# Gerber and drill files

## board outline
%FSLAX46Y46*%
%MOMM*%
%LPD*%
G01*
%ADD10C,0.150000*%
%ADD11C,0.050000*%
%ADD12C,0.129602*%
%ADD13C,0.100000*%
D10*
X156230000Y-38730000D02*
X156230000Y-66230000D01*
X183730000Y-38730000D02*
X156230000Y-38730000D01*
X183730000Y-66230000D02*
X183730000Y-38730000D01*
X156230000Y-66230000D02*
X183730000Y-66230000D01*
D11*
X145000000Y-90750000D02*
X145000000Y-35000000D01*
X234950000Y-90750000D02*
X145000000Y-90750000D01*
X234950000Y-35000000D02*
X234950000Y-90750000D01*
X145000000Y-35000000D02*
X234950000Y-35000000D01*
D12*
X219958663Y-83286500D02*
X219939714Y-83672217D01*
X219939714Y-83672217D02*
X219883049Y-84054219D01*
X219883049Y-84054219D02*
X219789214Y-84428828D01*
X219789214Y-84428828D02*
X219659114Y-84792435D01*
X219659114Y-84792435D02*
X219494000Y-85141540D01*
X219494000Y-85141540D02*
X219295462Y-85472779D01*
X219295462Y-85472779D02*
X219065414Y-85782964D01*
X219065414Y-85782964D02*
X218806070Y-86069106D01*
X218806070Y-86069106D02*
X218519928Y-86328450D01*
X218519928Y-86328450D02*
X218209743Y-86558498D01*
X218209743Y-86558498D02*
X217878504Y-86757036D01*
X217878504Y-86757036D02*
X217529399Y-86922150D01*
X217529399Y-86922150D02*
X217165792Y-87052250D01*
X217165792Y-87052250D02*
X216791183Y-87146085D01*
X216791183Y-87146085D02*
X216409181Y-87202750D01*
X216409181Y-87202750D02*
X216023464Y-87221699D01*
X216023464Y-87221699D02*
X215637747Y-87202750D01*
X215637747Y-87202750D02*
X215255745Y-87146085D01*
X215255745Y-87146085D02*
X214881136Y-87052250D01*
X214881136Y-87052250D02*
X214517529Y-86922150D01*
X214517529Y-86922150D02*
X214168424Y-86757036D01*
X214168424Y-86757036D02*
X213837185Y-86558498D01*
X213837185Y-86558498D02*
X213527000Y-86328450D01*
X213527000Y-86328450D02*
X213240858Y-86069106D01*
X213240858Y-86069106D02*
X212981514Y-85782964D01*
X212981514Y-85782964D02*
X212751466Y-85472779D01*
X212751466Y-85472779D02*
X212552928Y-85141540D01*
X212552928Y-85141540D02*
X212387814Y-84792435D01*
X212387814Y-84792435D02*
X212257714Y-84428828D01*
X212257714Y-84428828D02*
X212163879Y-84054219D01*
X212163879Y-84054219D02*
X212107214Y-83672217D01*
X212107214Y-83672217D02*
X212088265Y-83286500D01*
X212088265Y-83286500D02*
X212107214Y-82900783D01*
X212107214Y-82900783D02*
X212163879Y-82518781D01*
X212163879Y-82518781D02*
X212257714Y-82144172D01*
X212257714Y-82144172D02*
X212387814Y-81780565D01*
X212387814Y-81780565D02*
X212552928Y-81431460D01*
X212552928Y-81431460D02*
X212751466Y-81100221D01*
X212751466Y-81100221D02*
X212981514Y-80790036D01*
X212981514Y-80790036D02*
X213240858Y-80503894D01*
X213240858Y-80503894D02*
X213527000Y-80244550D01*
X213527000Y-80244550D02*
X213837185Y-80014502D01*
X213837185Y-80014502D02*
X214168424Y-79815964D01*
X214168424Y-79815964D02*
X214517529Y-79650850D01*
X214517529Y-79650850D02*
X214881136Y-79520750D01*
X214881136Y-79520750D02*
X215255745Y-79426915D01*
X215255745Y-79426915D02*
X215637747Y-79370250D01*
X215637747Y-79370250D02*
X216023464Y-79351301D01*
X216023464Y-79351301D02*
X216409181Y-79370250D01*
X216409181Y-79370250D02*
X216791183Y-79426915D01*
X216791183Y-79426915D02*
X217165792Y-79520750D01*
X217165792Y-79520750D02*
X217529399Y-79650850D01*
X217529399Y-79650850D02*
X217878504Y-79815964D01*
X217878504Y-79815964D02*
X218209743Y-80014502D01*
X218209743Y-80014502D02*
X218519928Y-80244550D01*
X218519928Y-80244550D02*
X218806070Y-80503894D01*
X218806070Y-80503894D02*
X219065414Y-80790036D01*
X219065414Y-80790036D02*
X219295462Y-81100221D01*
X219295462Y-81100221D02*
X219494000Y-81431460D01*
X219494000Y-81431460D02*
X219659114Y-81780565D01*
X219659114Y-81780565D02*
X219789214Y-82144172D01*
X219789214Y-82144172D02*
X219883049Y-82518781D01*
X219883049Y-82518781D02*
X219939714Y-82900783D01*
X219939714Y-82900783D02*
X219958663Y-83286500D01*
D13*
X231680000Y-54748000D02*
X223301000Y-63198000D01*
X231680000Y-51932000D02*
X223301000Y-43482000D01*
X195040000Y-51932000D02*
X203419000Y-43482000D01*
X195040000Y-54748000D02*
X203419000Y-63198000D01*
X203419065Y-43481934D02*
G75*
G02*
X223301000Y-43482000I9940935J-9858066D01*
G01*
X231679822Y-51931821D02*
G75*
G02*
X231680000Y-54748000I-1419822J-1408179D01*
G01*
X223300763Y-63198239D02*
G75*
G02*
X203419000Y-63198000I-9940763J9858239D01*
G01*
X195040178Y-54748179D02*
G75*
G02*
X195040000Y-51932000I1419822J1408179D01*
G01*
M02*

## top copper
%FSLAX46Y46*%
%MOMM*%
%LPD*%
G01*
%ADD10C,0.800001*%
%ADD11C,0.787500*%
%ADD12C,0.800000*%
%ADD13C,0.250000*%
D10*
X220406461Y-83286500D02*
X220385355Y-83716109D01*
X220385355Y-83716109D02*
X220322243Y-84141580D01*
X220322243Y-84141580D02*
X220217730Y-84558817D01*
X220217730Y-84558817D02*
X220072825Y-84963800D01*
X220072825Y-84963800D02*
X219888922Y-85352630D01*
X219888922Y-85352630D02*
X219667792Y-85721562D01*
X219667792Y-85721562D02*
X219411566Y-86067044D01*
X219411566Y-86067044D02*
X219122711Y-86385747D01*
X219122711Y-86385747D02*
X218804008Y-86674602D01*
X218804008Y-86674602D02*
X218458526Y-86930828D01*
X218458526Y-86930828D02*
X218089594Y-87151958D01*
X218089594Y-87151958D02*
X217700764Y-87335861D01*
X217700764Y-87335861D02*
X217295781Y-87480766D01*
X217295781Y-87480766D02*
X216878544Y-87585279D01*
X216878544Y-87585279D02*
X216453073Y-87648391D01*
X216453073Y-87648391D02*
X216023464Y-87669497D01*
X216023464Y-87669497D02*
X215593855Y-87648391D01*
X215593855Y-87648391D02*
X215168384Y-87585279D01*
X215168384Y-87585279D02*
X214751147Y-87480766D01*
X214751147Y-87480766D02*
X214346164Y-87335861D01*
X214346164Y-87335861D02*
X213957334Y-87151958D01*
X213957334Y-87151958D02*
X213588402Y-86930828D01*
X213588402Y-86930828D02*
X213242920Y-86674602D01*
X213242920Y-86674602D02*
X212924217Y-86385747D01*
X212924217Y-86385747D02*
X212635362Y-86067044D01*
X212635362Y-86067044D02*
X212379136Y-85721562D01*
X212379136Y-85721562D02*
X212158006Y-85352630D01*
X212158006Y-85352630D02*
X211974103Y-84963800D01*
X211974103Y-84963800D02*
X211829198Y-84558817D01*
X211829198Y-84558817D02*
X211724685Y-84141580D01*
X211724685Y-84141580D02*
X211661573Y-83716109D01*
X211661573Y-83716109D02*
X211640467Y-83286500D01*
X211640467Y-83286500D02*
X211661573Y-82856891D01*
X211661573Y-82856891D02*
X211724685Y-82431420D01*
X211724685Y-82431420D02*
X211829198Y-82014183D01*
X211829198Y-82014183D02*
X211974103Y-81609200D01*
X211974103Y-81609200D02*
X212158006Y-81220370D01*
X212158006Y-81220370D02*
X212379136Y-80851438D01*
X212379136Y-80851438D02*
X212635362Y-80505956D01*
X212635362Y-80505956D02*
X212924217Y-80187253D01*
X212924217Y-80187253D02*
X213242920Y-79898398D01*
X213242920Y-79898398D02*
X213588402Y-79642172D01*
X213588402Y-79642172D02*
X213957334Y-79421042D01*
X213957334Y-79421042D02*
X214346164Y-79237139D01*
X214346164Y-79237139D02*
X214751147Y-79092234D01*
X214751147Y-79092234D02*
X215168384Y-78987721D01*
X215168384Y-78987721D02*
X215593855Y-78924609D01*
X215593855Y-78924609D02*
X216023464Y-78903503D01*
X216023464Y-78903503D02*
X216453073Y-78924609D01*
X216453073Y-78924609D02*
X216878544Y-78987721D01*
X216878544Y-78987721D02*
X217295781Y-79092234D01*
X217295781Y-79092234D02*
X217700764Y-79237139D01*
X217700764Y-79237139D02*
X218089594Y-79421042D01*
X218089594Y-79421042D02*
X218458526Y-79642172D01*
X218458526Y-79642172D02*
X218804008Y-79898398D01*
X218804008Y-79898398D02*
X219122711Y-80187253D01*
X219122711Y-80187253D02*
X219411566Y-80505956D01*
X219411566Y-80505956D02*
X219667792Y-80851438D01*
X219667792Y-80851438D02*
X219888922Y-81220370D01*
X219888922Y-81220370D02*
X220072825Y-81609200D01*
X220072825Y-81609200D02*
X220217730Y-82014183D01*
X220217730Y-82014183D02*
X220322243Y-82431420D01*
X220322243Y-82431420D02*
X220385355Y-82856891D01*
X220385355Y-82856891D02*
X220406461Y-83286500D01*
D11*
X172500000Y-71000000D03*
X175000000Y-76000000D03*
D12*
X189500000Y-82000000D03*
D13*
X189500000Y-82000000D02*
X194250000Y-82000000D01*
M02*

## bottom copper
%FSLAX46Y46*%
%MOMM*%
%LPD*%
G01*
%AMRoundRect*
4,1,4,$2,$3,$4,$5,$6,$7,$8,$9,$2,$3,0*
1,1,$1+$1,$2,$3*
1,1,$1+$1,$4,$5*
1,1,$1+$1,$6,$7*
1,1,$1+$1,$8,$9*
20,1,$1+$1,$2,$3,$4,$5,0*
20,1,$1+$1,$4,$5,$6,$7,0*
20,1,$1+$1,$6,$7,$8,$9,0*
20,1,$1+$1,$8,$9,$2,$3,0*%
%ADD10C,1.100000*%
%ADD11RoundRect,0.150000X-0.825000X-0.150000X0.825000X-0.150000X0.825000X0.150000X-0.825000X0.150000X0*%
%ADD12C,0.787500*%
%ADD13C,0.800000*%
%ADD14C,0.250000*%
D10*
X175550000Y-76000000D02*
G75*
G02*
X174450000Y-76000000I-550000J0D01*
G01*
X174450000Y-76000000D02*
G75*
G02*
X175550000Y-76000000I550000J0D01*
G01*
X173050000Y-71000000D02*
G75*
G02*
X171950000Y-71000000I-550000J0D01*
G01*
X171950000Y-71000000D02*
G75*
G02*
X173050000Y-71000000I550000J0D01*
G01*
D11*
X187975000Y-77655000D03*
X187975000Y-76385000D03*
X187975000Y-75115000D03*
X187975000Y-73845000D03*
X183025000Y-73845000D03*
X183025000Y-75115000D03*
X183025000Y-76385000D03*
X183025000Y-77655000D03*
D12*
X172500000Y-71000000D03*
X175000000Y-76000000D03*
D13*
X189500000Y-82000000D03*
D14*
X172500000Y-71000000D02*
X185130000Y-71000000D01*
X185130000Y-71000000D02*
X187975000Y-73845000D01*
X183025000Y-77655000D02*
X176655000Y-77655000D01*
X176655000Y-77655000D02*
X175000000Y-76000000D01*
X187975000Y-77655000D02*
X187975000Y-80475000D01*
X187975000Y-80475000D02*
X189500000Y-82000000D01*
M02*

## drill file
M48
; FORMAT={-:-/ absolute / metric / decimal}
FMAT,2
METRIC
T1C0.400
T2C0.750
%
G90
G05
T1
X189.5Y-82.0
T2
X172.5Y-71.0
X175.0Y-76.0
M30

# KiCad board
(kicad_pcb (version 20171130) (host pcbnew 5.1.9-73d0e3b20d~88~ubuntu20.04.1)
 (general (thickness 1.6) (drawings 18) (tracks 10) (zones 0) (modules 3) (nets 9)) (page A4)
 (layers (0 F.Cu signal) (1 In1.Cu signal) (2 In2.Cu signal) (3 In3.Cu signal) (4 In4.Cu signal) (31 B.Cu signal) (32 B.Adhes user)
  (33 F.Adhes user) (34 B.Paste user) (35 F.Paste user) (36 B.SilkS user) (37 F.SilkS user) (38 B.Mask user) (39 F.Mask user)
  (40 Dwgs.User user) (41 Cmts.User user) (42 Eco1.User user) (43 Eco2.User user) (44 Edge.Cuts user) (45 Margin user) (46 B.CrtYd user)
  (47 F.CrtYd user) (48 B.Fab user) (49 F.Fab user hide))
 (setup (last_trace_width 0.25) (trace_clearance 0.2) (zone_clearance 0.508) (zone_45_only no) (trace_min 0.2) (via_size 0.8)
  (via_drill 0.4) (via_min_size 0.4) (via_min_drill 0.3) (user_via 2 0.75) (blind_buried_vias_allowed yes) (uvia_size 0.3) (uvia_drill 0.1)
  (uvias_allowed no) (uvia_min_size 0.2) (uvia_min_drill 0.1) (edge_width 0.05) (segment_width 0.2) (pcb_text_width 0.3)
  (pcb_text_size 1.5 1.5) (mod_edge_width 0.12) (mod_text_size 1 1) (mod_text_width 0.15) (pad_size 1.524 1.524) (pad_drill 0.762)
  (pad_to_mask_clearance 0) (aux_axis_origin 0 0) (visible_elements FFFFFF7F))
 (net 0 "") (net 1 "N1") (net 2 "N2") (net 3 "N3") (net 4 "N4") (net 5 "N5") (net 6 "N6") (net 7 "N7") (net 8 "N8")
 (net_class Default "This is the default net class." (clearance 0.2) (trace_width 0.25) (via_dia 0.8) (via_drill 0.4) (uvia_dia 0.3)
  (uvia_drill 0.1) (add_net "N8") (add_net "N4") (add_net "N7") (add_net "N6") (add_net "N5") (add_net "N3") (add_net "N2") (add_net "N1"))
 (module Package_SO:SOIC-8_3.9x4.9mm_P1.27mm (layer B.Cu) (at 185.5 75.75)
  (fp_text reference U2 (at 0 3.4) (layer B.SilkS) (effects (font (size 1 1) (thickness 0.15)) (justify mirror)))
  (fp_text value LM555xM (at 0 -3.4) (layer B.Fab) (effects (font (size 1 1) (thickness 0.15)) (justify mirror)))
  (pad 8 smd roundrect (at 2.475 1.905) (size 1.95 0.6) (layers B.Cu B.Paste B.Mask) (roundrect_rratio 0.25) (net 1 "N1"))
  (pad 7 smd roundrect (at 2.475 0.635) (size 1.95 0.6) (layers B.Cu B.Paste B.Mask) (roundrect_rratio 0.25) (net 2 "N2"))
  (pad 6 smd roundrect (at 2.475 -0.635) (size 1.95 0.6) (layers B.Cu B.Paste B.Mask) (roundrect_rratio 0.25) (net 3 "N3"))
  (pad 5 smd roundrect (at 2.475 -1.905) (size 1.95 0.6) (layers B.Cu B.Paste B.Mask) (roundrect_rratio 0.25) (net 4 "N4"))
  (pad 4 smd roundrect (at -2.475 -1.905) (size 1.95 0.6) (layers B.Cu B.Paste B.Mask) (roundrect_rratio 0.25) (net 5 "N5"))
  (pad 3 smd roundrect (at -2.475 -0.635) (size 1.95 0.6) (layers B.Cu B.Paste B.Mask) (roundrect_rratio 0.25) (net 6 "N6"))
  (pad 2 smd roundrect (at -2.475 0.635) (size 1.95 0.6) (layers B.Cu B.Paste B.Mask) (roundrect_rratio 0.25) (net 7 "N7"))
  (pad 1 smd roundrect (at -2.475 1.905) (size 1.95 0.6) (layers B.Cu B.Paste B.Mask) (roundrect_rratio 0.25) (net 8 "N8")))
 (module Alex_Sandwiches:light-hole (layer F.Cu) (at 201.93 77.47)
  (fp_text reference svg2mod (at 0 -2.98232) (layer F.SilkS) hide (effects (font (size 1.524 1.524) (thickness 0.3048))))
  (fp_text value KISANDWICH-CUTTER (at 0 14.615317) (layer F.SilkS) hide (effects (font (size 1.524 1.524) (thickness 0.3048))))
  (fp_line (start 18.476461 5.8165) (end 18.455355 6.246109) (layer F.Cu) (width 0.800001))
  (fp_line (start 18.455355 6.246109) (end 18.392243 6.67158) (layer F.Cu) (width 0.800001))
  (fp_line (start 18.392243 6.67158) (end 18.28773 7.088817) (layer F.Cu) (width 0.800001))
  (fp_line (start 18.28773 7.088817) (end 18.142825 7.4938) (layer F.Cu) (width 0.800001))
  (fp_line (start 18.142825 7.4938) (end 17.958922 7.88263) (layer F.Cu) (width 0.800001))
  (fp_line (start 17.958922 7.88263) (end 17.737792 8.251562) (layer F.Cu) (width 0.800001))
  (fp_line (start 17.737792 8.251562) (end 17.481566 8.597044) (layer F.Cu) (width 0.800001))
  (fp_line (start 17.481566 8.597044) (end 17.192711 8.915747) (layer F.Cu) (width 0.800001))
  (fp_line (start 17.192711 8.915747) (end 16.874008 9.204602) (layer F.Cu) (width 0.800001))
  (fp_line (start 16.874008 9.204602) (end 16.528526 9.460828) (layer F.Cu) (width 0.800001))
  (fp_line (start 16.528526 9.460828) (end 16.159594 9.681958) (layer F.Cu) (width 0.800001))
  (fp_line (start 16.159594 9.681958) (end 15.770764 9.865861) (layer F.Cu) (width 0.800001))
  (fp_line (start 15.770764 9.865861) (end 15.365781 10.010766) (layer F.Cu) (width 0.800001))
  (fp_line (start 15.365781 10.010766) (end 14.948544 10.115279) (layer F.Cu) (width 0.800001))
  (fp_line (start 14.948544 10.115279) (end 14.523073 10.178391) (layer F.Cu) (width 0.800001))
  (fp_line (start 14.523073 10.178391) (end 14.093464 10.199497) (layer F.Cu) (width 0.800001))
  (fp_line (start 14.093464 10.199497) (end 13.663855 10.178391) (layer F.Cu) (width 0.800001))
  (fp_line (start 13.663855 10.178391) (end 13.238384 10.115279) (layer F.Cu) (width 0.800001))
  (fp_line (start 13.238384 10.115279) (end 12.821147 10.010766) (layer F.Cu) (width 0.800001))
  (fp_line (start 12.821147 10.010766) (end 12.416164 9.865861) (layer F.Cu) (width 0.800001))
  (fp_line (start 12.416164 9.865861) (end 12.027334 9.681958) (layer F.Cu) (width 0.800001))
  (fp_line (start 12.027334 9.681958) (end 11.658402 9.460828) (layer F.Cu) (width 0.800001))
  (fp_line (start 11.658402 9.460828) (end 11.31292 9.204602) (layer F.Cu) (width 0.800001))
  (fp_line (start 11.31292 9.204602) (end 10.994217 8.915747) (layer F.Cu) (width 0.800001))
  (fp_line (start 10.994217 8.915747) (end 10.705362 8.597044) (layer F.Cu) (width 0.800001))
  (fp_line (start 10.705362 8.597044) (end 10.449136 8.251562) (layer F.Cu) (width 0.800001))
  (fp_line (start 10.449136 8.251562) (end 10.228006 7.88263) (layer F.Cu) (width 0.800001))
  (fp_line (start 10.228006 7.88263) (end 10.044103 7.4938) (layer F.Cu) (width 0.800001))
  (fp_line (start 10.044103 7.4938) (end 9.899198 7.088817) (layer F.Cu) (width 0.800001))
  (fp_line (start 9.899198 7.088817) (end 9.794685 6.67158) (layer F.Cu) (width 0.800001))
  (fp_line (start 9.794685 6.67158) (end 9.731573 6.246109) (layer F.Cu) (width 0.800001))
  (fp_line (start 9.731573 6.246109) (end 9.710467 5.8165) (layer F.Cu) (width 0.800001))
  (fp_line (start 9.710467 5.8165) (end 9.731573 5.386891) (layer F.Cu) (width 0.800001))
  (fp_line (start 9.731573 5.386891) (end 9.794685 4.96142) (layer F.Cu) (width 0.800001))
  (fp_line (start 9.794685 4.96142) (end 9.899198 4.544183) (layer F.Cu) (width 0.800001))
  (fp_line (start 9.899198 4.544183) (end 10.044103 4.1392) (layer F.Cu) (width 0.800001))
  (fp_line (start 10.044103 4.1392) (end 10.228006 3.75037) (layer F.Cu) (width 0.800001))
  (fp_line (start 10.228006 3.75037) (end 10.449136 3.381438) (layer F.Cu) (width 0.800001))
  (fp_line (start 10.449136 3.381438) (end 10.705362 3.035956) (layer F.Cu) (width 0.800001))
  (fp_line (start 10.705362 3.035956) (end 10.994217 2.717253) (layer F.Cu) (width 0.800001))
  (fp_line (start 10.994217 2.717253) (end 11.31292 2.428398) (layer F.Cu) (width 0.800001))
  (fp_line (start 11.31292 2.428398) (end 11.658402 2.172172) (layer F.Cu) (width 0.800001))
  (fp_line (start 11.658402 2.172172) (end 12.027334 1.951042) (layer F.Cu) (width 0.800001))
  (fp_line (start 12.027334 1.951042) (end 12.416164 1.767139) (layer F.Cu) (width 0.800001))
  (fp_line (start 12.416164 1.767139) (end 12.821147 1.622234) (layer F.Cu) (width 0.800001))
  (fp_line (start 12.821147 1.622234) (end 13.238384 1.517721) (layer F.Cu) (width 0.800001))
  (fp_line (start 13.238384 1.517721) (end 13.663855 1.454609) (layer F.Cu) (width 0.800001))
  (fp_line (start 13.663855 1.454609) (end 14.093464 1.433503) (layer F.Cu) (width 0.800001))
  (fp_line (start 14.093464 1.433503) (end 14.523073 1.454609) (layer F.Cu) (width 0.800001))
  (fp_line (start 14.523073 1.454609) (end 14.948544 1.517721) (layer F.Cu) (width 0.800001))
  (fp_line (start 14.948544 1.517721) (end 15.365781 1.622234) (layer F.Cu) (width 0.800001))
  (fp_line (start 15.365781 1.622234) (end 15.770764 1.767139) (layer F.Cu) (width 0.800001))
  (fp_line (start 15.770764 1.767139) (end 16.159594 1.951042) (layer F.Cu) (width 0.800001))
  (fp_line (start 16.159594 1.951042) (end 16.528526 2.172172) (layer F.Cu) (width 0.800001))
  (fp_line (start 16.528526 2.172172) (end 16.874008 2.428398) (layer F.Cu) (width 0.800001))
  (fp_line (start 16.874008 2.428398) (end 17.192711 2.717253) (layer F.Cu) (width 0.800001))
  (fp_line (start 17.192711 2.717253) (end 17.481566 3.035956) (layer F.Cu) (width 0.800001))
  (fp_line (start 17.481566 3.035956) (end 17.737792 3.381438) (layer F.Cu) (width 0.800001))
  (fp_line (start 17.737792 3.381438) (end 17.958922 3.75037) (layer F.Cu) (width 0.800001))
  (fp_line (start 17.958922 3.75037) (end 18.142825 4.1392) (layer F.Cu) (width 0.800001))
  (fp_line (start 18.142825 4.1392) (end 18.28773 4.544183) (layer F.Cu) (width 0.800001))
  (fp_line (start 18.28773 4.544183) (end 18.392243 4.96142) (layer F.Cu) (width 0.800001))
  (fp_line (start 18.392243 4.96142) (end 18.455355 5.386891) (layer F.Cu) (width 0.800001))
  (fp_line (start 18.455355 5.386891) (end 18.476461 5.8165) (layer F.Cu) (width 0.800001))
  (fp_line (start 18.028663 5.8165) (end 18.009714 6.202217) (layer Edge.Cuts) (width 0.129602))
  (fp_line (start 18.009714 6.202217) (end 17.953049 6.584219) (layer Edge.Cuts) (width 0.129602))
  (fp_line (start 17.953049 6.584219) (end 17.859214 6.958828) (layer Edge.Cuts) (width 0.129602))
  (fp_line (start 17.859214 6.958828) (end 17.729114 7.322435) (layer Edge.Cuts) (width 0.129602))
  (fp_line (start 17.729114 7.322435) (end 17.564 7.67154) (layer Edge.Cuts) (width 0.129602))
  (fp_line (start 17.564 7.67154) (end 17.365462 8.002779) (layer Edge.Cuts) (width 0.129602))
  (fp_line (start 17.365462 8.002779) (end 17.135414 8.312964) (layer Edge.Cuts) (width 0.129602))
  (fp_line (start 17.135414 8.312964) (end 16.87607 8.599106) (layer Edge.Cuts) (width 0.129602))
  (fp_line (start 16.87607 8.599106) (end 16.589928 8.85845) (layer Edge.Cuts) (width 0.129602))
  (fp_line (start 16.589928 8.85845) (end 16.279743 9.088498) (layer Edge.Cuts) (width 0.129602))
  (fp_line (start 16.279743 9.088498) (end 15.948504 9.287036) (layer Edge.Cuts) (width 0.129602))
  (fp_line (start 15.948504 9.287036) (end 15.599399 9.45215) (layer Edge.Cuts) (width 0.129602))
  (fp_line (start 15.599399 9.45215) (end 15.235792 9.58225) (layer Edge.Cuts) (width 0.129602))
  (fp_line (start 15.235792 9.58225) (end 14.861183 9.676085) (layer Edge.Cuts) (width 0.129602))
  (fp_line (start 14.861183 9.676085) (end 14.479181 9.73275) (layer Edge.Cuts) (width 0.129602))
  (fp_line (start 14.479181 9.73275) (end 14.093464 9.751699) (layer Edge.Cuts) (width 0.129602))
  (fp_line (start 14.093464 9.751699) (end 13.707747 9.73275) (layer Edge.Cuts) (width 0.129602))
  (fp_line (start 13.707747 9.73275) (end 13.325745 9.676085) (layer Edge.Cuts) (width 0.129602))
  (fp_line (start 13.325745 9.676085) (end 12.951136 9.58225) (layer Edge.Cuts) (width 0.129602))
  (fp_line (start 12.951136 9.58225) (end 12.587529 9.45215) (layer Edge.Cuts) (width 0.129602))
  (fp_line (start 12.587529 9.45215) (end 12.238424 9.287036) (layer Edge.Cuts) (width 0.129602))
  (fp_line (start 12.238424 9.287036) (end 11.907185 9.088498) (layer Edge.Cuts) (width 0.129602))
  (fp_line (start 11.907185 9.088498) (end 11.597 8.85845) (layer Edge.Cuts) (width 0.129602))
  (fp_line (start 11.597 8.85845) (end 11.310858 8.599106) (layer Edge.Cuts) (width 0.129602))
  (fp_line (start 11.310858 8.599106) (end 11.051514 8.312964) (layer Edge.Cuts) (width 0.129602))
  (fp_line (start 11.051514 8.312964) (end 10.821466 8.002779) (layer Edge.Cuts) (width 0.129602))
  (fp_line (start 10.821466 8.002779) (end 10.622928 7.67154) (layer Edge.Cuts) (width 0.129602))
  (fp_line (start 10.622928 7.67154) (end 10.457814 7.322435) (layer Edge.Cuts) (width 0.129602))
  (fp_line (start 10.457814 7.322435) (end 10.327714 6.958828) (layer Edge.Cuts) (width 0.129602))
  (fp_line (start 10.327714 6.958828) (end 10.233879 6.584219) (layer Edge.Cuts) (width 0.129602))
  (fp_line (start 10.233879 6.584219) (end 10.177214 6.202217) (layer Edge.Cuts) (width 0.129602))
  (fp_line (start 10.177214 6.202217) (end 10.158265 5.8165) (layer Edge.Cuts) (width 0.129602))
  (fp_line (start 10.158265 5.8165) (end 10.177214 5.430783) (layer Edge.Cuts) (width 0.129602))
  (fp_line (start 10.177214 5.430783) (end 10.233879 5.048781) (layer Edge.Cuts) (width 0.129602))
  (fp_line (start 10.233879 5.048781) (end 10.327714 4.674172) (layer Edge.Cuts) (width 0.129602))
  (fp_line (start 10.327714 4.674172) (end 10.457814 4.310565) (layer Edge.Cuts) (width 0.129602))
  (fp_line (start 10.457814 4.310565) (end 10.622928 3.96146) (layer Edge.Cuts) (width 0.129602))
  (fp_line (start 10.622928 3.96146) (end 10.821466 3.630221) (layer Edge.Cuts) (width 0.129602))
  (fp_line (start 10.821466 3.630221) (end 11.051514 3.320036) (layer Edge.Cuts) (width 0.129602))
  (fp_line (start 11.051514 3.320036) (end 11.310858 3.033894) (layer Edge.Cuts) (width 0.129602))
  (fp_line (start 11.310858 3.033894) (end 11.597 2.77455) (layer Edge.Cuts) (width 0.129602))
  (fp_line (start 11.597 2.77455) (end 11.907185 2.544502) (layer Edge.Cuts) (width 0.129602))
  (fp_line (start 11.907185 2.544502) (end 12.238424 2.345964) (layer Edge.Cuts) (width 0.129602))
  (fp_line (start 12.238424 2.345964) (end 12.587529 2.18085) (layer Edge.Cuts) (width 0.129602))
  (fp_line (start 12.587529 2.18085) (end 12.951136 2.05075) (layer Edge.Cuts) (width 0.129602))
  (fp_line (start 12.951136 2.05075) (end 13.325745 1.956915) (layer Edge.Cuts) (width 0.129602))
  (fp_line (start 13.325745 1.956915) (end 13.707747 1.90025) (layer Edge.Cuts) (width 0.129602))
  (fp_line (start 13.707747 1.90025) (end 14.093464 1.881301) (layer Edge.Cuts) (width 0.129602))
  (fp_line (start 14.093464 1.881301) (end 14.479181 1.90025) (layer Edge.Cuts) (width 0.129602))
  (fp_line (start 14.479181 1.90025) (end 14.861183 1.956915) (layer Edge.Cuts) (width 0.129602))
  (fp_line (start 14.861183 1.956915) (end 15.235792 2.05075) (layer Edge.Cuts) (width 0.129602))
  (fp_line (start 15.235792 2.05075) (end 15.599399 2.18085) (layer Edge.Cuts) (width 0.129602))
  (fp_line (start 15.599399 2.18085) (end 15.948504 2.345964) (layer Edge.Cuts) (width 0.129602))
  (fp_line (start 15.948504 2.345964) (end 16.279743 2.544502) (layer Edge.Cuts) (width 0.129602))
  (fp_line (start 16.279743 2.544502) (end 16.589928 2.77455) (layer Edge.Cuts) (width 0.129602))
  (fp_line (start 16.589928 2.77455) (end 16.87607 3.033894) (layer Edge.Cuts) (width 0.129602))
  (fp_line (start 16.87607 3.033894) (end 17.135414 3.320036) (layer Edge.Cuts) (width 0.129602))
  (fp_line (start 17.135414 3.320036) (end 17.365462 3.630221) (layer Edge.Cuts) (width 0.129602))
  (fp_line (start 17.365462 3.630221) (end 17.564 3.96146) (layer Edge.Cuts) (width 0.129602))
  (fp_line (start 17.564 3.96146) (end 17.729114 4.310565) (layer Edge.Cuts) (width 0.129602))
  (fp_line (start 17.729114 4.310565) (end 17.859214 4.674172) (layer Edge.Cuts) (width 0.129602))
  (fp_line (start 17.859214 4.674172) (end 17.953049 5.048781) (layer Edge.Cuts) (width 0.129602))
  (fp_line (start 17.953049 5.048781) (end 18.009714 5.430783) (layer Edge.Cuts) (width 0.129602))
  (fp_line (start 18.009714 5.430783) (end 18.028663 5.8165) (layer Edge.Cuts) (width 0.129602)))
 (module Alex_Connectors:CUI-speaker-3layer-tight (layer F.Cu) (at 213.36 53.34 180)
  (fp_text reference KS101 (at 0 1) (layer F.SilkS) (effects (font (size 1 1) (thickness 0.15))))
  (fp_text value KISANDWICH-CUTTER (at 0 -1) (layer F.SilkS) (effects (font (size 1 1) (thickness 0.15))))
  (fp_line (start -18.32 -1.408) (end -9.941 -9.858) (layer Edge.Cuts) (width 0.1))
  (fp_line (start -18.32 1.408) (end -9.941 9.858) (layer Edge.Cuts) (width 0.1))
  (fp_line (start 18.32 1.408) (end 9.941 9.858) (layer Edge.Cuts) (width 0.1))
  (fp_line (start 18.32 -1.408) (end 9.941 -9.858) (layer Edge.Cuts) (width 0.1))
  (fp_arc (start 0 0) (end -9.941 9.858) (angle -90.48) (layer Edge.Cuts) (width 0.1))
  (fp_arc (start -16.9 0) (end -18.32 -1.408) (angle -89.521) (layer Edge.Cuts) (width 0.1))
  (fp_arc (start 0 0) (end 9.941 -9.858) (angle -90.479) (layer Edge.Cuts) (width 0.1))
  (fp_arc (start 16.9 0) (end 18.32 1.408) (angle -89.521) (layer Edge.Cuts) (width 0.1)))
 (gr_circle (center 175 76) (end 175 76.55) (layer B.Cu) (width 1.1))
 (gr_circle (center 172.5 71) (end 172.5 71.55) (layer B.Cu) (width 1.1))
 (gr_line (start 156.23 38.73) (end 156.23 66.23) (layer Edge.Cuts) (width 0.15))
 (gr_line (start 183.73 38.73) (end 156.23 38.73) (layer Edge.Cuts) (width 0.15))
 (gr_line (start 183.73 66.23) (end 183.73 38.73) (layer Edge.Cuts) (width 0.15))
 (gr_line (start 156.23 66.23) (end 183.73 66.23) (layer Edge.Cuts) (width 0.15))
 (gr_line (start 145 90.75) (end 145 35) (layer Edge.Cuts) (width 0.05))
 (gr_line (start 234.95 90.75) (end 145 90.75) (layer Edge.Cuts) (width 0.05))
 (gr_line (start 234.95 35) (end 234.95 90.75) (layer Edge.Cuts) (width 0.05))
 (gr_line (start 145 35) (end 234.95 35) (layer Edge.Cuts) (width 0.05))
 (via (at 172.5 71) (size 0.7875) (drill 0.75) (layers F.Cu B.Cu) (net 4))
 (segment (start 172.5 71) (end 185.13 71) (width 0.25) (layer B.Cu) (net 4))
 (segment (start 185.13 71) (end 187.975 73.845) (width 0.25) (layer B.Cu) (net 4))
 (via (at 175 76) (size 0.7875) (drill 0.75) (layers F.Cu B.Cu) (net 8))
 (segment (start 183.025 77.655) (end 176.655 77.655) (width 0.25) (layer B.Cu) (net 8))
 (segment (start 176.655 77.655) (end 175 76) (width 0.25) (layer B.Cu) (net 8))
 (segment (start 189.5 82) (end 194.25 82) (width 0.25) (layer F.Cu) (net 1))
 (segment (start 187.975 77.655) (end 187.975 80.475) (width 0.25) (layer B.Cu) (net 1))
 (segment (start 187.975 80.475) (end 189.5 82) (width 0.25) (layer B.Cu) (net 1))
 (via (at 189.5 82) (size 0.8) (drill 0.4) (layers F.Cu B.Cu) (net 1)))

